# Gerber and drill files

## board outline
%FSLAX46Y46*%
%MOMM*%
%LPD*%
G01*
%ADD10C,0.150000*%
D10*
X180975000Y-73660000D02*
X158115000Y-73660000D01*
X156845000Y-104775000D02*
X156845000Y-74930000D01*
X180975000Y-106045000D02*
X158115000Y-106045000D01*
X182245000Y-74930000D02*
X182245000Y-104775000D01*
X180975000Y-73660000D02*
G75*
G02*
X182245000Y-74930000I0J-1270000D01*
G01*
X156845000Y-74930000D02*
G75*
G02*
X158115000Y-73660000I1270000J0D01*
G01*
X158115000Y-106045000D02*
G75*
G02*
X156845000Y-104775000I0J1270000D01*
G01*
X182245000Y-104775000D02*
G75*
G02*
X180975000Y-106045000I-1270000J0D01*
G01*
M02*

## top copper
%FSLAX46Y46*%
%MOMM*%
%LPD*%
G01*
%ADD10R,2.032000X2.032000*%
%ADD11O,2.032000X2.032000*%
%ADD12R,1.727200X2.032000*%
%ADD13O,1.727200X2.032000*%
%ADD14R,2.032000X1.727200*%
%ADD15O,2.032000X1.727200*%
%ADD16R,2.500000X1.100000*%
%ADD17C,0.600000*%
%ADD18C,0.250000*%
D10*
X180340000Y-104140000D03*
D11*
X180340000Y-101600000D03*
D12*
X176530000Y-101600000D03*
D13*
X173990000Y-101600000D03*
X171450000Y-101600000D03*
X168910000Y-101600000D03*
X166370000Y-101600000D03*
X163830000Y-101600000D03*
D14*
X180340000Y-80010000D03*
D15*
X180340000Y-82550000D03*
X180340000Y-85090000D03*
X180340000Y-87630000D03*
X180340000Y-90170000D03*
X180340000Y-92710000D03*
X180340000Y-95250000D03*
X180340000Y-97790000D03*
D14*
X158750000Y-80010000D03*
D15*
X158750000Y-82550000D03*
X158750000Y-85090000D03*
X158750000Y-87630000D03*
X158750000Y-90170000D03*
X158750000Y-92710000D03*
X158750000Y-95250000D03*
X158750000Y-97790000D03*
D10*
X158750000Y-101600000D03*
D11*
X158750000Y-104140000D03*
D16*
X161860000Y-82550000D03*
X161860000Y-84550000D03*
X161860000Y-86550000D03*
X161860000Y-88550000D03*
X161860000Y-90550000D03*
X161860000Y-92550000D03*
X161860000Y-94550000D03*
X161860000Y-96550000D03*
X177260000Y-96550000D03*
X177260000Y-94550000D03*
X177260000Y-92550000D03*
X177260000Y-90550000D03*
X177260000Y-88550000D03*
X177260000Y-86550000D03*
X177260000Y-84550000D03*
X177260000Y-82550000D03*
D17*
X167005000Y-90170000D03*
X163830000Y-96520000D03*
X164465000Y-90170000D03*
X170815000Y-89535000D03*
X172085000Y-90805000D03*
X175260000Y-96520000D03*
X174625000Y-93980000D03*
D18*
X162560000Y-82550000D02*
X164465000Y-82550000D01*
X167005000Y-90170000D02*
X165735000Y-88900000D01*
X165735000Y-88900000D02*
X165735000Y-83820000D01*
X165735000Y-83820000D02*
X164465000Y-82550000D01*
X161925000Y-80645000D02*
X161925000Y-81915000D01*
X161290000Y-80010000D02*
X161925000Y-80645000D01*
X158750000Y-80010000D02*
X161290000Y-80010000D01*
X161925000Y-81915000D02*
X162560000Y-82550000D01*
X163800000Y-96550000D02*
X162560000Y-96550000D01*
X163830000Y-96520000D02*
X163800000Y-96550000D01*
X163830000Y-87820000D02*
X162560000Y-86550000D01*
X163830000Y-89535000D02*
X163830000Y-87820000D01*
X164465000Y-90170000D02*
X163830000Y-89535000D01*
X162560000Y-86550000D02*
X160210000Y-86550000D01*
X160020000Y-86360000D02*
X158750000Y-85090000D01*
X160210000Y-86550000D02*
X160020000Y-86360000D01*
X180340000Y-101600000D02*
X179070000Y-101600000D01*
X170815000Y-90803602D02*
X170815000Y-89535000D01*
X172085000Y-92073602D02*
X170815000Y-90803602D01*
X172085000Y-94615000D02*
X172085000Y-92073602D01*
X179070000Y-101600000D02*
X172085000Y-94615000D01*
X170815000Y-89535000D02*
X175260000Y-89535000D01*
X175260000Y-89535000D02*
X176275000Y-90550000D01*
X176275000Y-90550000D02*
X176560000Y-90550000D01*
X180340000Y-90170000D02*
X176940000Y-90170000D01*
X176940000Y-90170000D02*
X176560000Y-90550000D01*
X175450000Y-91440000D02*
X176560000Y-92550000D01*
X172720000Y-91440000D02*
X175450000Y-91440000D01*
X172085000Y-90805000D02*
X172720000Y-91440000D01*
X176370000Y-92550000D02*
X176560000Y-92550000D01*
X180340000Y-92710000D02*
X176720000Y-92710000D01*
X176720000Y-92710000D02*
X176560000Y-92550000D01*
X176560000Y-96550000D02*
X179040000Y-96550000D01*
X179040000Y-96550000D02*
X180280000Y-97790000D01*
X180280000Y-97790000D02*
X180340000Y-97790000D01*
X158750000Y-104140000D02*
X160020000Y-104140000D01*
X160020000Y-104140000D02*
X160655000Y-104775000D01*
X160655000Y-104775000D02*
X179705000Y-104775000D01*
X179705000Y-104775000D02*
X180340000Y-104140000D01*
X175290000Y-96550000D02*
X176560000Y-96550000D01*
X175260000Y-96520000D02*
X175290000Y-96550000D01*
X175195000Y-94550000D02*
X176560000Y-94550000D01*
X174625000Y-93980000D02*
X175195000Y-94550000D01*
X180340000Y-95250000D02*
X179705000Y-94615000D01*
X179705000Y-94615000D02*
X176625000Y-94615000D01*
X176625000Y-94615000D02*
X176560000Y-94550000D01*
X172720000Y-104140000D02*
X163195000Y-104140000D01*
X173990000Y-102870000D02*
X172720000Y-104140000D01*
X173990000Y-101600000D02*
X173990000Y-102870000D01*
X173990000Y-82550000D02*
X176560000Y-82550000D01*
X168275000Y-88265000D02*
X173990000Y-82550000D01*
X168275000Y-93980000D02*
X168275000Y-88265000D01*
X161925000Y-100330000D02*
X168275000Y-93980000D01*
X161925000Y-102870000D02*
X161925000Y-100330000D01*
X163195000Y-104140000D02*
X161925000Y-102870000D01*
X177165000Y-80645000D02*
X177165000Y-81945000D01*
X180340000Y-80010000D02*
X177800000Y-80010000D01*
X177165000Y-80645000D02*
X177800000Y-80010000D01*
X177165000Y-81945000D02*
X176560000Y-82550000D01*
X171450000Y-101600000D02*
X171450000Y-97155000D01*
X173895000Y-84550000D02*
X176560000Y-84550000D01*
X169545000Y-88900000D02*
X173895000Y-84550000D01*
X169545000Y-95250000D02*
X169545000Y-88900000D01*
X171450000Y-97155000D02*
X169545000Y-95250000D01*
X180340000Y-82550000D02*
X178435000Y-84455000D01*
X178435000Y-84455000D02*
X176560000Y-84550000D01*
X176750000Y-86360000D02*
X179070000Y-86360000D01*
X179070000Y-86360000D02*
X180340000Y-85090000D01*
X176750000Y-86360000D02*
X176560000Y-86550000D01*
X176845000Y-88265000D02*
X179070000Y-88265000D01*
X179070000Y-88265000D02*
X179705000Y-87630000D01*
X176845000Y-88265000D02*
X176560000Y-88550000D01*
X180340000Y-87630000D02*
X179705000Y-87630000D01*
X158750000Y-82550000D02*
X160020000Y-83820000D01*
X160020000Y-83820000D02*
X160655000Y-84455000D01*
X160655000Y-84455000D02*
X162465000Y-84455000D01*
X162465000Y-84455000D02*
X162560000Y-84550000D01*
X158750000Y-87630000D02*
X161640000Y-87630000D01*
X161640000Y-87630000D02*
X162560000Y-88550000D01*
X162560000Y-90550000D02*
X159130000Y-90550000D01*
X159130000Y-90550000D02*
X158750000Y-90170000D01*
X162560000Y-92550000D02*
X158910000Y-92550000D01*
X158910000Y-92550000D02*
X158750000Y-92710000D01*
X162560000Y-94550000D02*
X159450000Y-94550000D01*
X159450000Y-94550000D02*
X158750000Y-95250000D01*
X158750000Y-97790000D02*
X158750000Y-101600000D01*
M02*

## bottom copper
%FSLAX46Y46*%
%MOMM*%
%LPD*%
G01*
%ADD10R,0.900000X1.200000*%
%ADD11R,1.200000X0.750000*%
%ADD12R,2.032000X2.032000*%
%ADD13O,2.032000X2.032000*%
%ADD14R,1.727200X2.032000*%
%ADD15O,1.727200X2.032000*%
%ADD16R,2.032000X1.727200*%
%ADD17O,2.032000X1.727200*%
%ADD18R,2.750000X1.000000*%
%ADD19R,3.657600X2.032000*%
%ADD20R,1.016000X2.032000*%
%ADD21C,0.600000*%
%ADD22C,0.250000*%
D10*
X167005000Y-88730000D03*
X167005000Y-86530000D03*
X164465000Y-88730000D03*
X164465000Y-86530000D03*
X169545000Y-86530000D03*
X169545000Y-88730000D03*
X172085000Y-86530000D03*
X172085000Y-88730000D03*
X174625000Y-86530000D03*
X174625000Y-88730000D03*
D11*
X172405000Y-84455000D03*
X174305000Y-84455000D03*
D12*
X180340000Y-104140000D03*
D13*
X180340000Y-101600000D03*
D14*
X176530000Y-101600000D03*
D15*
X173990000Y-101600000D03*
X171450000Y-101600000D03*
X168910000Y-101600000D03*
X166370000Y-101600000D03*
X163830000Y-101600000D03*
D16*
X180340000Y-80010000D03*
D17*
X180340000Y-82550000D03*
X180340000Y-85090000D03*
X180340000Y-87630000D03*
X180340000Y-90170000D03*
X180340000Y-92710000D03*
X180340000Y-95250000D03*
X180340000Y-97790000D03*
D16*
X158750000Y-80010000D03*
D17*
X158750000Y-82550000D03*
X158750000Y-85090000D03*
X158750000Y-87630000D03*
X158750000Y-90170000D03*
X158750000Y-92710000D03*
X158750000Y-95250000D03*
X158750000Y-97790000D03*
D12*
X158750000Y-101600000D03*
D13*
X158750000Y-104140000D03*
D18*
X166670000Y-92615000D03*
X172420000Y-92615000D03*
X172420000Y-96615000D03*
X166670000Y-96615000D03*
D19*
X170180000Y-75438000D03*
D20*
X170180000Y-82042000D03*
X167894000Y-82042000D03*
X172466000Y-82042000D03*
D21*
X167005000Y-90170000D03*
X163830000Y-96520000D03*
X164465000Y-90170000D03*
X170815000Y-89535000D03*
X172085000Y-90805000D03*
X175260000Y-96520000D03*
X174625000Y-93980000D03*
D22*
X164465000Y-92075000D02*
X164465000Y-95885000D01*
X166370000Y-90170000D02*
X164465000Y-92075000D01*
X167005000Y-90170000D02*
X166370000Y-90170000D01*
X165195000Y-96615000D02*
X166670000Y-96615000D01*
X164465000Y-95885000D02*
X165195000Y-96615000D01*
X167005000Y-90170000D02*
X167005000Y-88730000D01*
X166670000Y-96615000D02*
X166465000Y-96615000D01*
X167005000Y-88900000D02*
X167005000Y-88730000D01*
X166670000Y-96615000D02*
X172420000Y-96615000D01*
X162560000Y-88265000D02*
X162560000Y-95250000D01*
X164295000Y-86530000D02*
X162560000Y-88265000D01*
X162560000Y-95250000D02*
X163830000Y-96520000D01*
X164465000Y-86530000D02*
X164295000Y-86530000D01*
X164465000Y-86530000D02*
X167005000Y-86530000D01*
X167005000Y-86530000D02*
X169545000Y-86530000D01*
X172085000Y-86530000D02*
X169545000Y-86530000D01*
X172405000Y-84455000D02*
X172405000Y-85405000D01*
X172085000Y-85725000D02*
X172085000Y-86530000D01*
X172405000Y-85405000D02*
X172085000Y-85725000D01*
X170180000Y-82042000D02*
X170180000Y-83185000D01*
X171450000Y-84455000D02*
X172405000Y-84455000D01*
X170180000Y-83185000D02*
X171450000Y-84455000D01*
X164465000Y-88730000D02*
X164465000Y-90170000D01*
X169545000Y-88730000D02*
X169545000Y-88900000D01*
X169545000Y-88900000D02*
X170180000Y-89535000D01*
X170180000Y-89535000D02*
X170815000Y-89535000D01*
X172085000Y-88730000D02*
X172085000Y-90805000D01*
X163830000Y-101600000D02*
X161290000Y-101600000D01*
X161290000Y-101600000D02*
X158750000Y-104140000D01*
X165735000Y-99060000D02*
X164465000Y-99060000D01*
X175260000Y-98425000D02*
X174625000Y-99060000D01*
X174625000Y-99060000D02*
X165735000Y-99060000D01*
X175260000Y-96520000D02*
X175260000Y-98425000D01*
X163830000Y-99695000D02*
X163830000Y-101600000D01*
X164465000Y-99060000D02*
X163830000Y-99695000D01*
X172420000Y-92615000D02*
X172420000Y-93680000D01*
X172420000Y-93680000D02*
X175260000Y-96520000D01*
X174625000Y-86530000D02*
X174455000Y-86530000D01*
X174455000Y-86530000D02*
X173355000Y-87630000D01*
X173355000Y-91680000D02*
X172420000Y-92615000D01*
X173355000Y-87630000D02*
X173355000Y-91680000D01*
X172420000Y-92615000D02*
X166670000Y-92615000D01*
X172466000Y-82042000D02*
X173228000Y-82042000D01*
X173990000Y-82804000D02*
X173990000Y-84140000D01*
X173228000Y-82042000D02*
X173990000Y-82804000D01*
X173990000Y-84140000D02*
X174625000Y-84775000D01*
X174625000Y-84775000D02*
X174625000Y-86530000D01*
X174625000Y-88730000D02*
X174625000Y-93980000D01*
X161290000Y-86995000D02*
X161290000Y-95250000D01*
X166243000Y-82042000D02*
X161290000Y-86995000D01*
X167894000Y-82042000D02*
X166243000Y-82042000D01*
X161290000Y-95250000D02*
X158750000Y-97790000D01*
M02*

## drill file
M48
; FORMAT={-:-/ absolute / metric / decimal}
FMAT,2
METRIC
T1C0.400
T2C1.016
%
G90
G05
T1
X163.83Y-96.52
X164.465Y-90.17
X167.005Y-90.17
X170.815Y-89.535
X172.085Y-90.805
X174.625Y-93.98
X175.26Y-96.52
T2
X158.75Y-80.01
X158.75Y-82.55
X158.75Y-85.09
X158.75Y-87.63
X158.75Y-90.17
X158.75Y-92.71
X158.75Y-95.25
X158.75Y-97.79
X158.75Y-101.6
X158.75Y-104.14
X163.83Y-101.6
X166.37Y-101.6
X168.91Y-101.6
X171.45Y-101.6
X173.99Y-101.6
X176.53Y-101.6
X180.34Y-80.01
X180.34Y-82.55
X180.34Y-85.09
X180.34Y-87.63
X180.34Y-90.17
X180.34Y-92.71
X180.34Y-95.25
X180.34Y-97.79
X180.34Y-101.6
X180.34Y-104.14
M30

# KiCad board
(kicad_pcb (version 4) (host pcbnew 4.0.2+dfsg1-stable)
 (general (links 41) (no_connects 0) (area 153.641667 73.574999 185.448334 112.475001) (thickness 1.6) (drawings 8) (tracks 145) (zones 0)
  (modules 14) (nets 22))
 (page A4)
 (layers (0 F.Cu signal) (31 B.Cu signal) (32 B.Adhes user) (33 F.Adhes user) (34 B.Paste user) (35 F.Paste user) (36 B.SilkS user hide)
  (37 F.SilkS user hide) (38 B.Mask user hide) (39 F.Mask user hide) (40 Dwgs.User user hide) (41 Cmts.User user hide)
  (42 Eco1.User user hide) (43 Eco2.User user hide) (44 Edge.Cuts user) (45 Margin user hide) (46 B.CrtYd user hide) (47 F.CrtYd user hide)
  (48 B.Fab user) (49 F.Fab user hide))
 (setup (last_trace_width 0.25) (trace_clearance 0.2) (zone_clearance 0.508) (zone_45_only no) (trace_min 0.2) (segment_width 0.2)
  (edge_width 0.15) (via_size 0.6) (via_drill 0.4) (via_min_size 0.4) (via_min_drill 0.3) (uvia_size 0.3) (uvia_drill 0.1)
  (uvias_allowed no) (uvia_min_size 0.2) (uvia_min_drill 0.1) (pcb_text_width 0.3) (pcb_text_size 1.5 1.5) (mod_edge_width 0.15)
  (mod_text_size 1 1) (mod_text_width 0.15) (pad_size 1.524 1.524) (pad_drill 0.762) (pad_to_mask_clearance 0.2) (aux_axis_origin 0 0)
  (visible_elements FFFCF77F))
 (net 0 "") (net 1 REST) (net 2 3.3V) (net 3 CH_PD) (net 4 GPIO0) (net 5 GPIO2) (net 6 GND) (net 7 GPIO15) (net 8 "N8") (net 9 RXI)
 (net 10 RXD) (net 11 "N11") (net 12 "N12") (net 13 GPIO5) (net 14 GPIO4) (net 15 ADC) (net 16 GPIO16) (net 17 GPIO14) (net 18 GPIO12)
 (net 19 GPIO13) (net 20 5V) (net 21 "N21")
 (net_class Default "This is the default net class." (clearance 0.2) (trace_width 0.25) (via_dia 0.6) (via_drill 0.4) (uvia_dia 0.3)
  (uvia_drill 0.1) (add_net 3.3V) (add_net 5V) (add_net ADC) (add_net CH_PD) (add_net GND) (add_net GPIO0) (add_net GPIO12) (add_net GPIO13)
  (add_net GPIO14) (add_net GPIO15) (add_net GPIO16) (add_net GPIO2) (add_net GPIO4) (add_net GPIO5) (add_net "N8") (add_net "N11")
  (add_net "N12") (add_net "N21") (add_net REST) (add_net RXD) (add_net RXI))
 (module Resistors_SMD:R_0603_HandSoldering (layer B.Cu) (at 167.005 87.63 90)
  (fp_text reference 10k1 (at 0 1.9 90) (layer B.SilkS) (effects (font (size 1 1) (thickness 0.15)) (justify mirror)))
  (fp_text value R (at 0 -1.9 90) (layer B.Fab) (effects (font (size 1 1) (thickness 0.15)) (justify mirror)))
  (pad 1 smd rect (at -1.1 0 90) (size 1.2 0.9) (layers B.Cu B.Paste B.Mask) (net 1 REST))
  (pad 2 smd rect (at 1.1 0 90) (size 1.2 0.9) (layers B.Cu B.Paste B.Mask) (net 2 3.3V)))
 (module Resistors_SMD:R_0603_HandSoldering (layer B.Cu) (at 164.465 87.63 90)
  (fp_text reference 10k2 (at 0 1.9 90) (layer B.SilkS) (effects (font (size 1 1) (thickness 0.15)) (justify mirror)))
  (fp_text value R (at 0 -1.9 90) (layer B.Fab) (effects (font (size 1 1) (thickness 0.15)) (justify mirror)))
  (pad 1 smd rect (at -1.1 0 90) (size 1.2 0.9) (layers B.Cu B.Paste B.Mask) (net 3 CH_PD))
  (pad 2 smd rect (at 1.1 0 90) (size 1.2 0.9) (layers B.Cu B.Paste B.Mask) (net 2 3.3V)))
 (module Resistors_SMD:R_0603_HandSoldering (layer B.Cu) (at 169.545 87.63 270)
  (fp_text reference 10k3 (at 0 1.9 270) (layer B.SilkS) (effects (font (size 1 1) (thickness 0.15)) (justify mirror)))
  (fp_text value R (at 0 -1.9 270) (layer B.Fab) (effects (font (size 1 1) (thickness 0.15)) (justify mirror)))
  (pad 1 smd rect (at -1.1 0 270) (size 1.2 0.9) (layers B.Cu B.Paste B.Mask) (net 2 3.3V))
  (pad 2 smd rect (at 1.1 0 270) (size 1.2 0.9) (layers B.Cu B.Paste B.Mask) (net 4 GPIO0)))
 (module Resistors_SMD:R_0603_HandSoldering (layer B.Cu) (at 172.085 87.63 270)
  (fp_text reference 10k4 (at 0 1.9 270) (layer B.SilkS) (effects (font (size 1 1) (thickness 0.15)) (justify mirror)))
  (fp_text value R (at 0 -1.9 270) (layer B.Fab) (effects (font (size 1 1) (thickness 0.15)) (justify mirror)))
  (pad 1 smd rect (at -1.1 0 270) (size 1.2 0.9) (layers B.Cu B.Paste B.Mask) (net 2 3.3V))
  (pad 2 smd rect (at 1.1 0 270) (size 1.2 0.9) (layers B.Cu B.Paste B.Mask) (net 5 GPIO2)))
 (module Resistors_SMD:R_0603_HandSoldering (layer B.Cu) (at 174.625 87.63 270)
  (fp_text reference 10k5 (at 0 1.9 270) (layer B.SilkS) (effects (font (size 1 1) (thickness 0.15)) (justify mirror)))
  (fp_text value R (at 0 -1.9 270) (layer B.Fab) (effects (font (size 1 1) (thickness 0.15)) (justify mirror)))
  (pad 1 smd rect (at -1.1 0 270) (size 1.2 0.9) (layers B.Cu B.Paste B.Mask) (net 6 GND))
  (pad 2 smd rect (at 1.1 0 270) (size 1.2 0.9) (layers B.Cu B.Paste B.Mask) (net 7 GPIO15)))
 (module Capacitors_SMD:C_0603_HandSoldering (layer B.Cu) (at 173.355 84.455)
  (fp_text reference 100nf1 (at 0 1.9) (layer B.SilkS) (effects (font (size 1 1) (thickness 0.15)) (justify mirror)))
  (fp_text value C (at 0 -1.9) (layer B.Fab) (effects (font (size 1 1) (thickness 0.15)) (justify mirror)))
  (pad 1 smd rect (at -0.95 0) (size 1.2 0.75) (layers B.Cu B.Paste B.Mask) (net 2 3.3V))
  (pad 2 smd rect (at 0.95 0) (size 1.2 0.75) (layers B.Cu B.Paste B.Mask) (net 6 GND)))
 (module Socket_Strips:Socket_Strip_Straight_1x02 (layer F.Cu) (at 180.34 104.14 90)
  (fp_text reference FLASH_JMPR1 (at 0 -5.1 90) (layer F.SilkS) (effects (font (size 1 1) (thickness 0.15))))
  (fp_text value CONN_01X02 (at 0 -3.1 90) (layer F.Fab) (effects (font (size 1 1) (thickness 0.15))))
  (pad 1 thru_hole rect (at 0 0 90) (size 2.032 2.032) (drill 1.016) (layers *.Cu *.Mask F.SilkS) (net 6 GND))
  (pad 2 thru_hole oval (at 2.54 0 90) (size 2.032 2.032) (drill 1.016) (layers *.Cu *.Mask F.SilkS) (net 4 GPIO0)))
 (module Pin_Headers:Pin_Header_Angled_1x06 (layer F.Cu) (at 176.53 101.6 270)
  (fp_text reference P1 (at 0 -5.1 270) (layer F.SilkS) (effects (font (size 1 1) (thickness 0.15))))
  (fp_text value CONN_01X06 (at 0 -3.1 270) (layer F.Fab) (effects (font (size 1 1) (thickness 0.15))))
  (pad 1 thru_hole rect (at 0 0 270) (size 2.032 1.7272) (drill 1.016) (layers *.Cu *.Mask F.SilkS) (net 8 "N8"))
  (pad 2 thru_hole oval (at 0 2.54 270) (size 2.032 1.7272) (drill 1.016) (layers *.Cu *.Mask F.SilkS) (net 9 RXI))
  (pad 3 thru_hole oval (at 0 5.08 270) (size 2.032 1.7272) (drill 1.016) (layers *.Cu *.Mask F.SilkS) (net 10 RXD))
  (pad 4 thru_hole oval (at 0 7.62 270) (size 2.032 1.7272) (drill 1.016) (layers *.Cu *.Mask F.SilkS) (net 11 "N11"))
  (pad 5 thru_hole oval (at 0 10.16 270) (size 2.032 1.7272) (drill 1.016) (layers *.Cu *.Mask F.SilkS) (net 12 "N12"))
  (pad 6 thru_hole oval (at 0 12.7 270) (size 2.032 1.7272) (drill 1.016) (layers *.Cu *.Mask F.SilkS) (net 6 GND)))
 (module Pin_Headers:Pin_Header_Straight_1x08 (layer F.Cu) (at 180.34 80.01)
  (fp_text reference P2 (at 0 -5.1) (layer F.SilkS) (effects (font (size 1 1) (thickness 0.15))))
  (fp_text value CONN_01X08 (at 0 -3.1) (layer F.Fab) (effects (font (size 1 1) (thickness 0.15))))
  (pad 1 thru_hole rect (at 0 0) (size 2.032 1.7272) (drill 1.016) (layers *.Cu *.Mask F.SilkS) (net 9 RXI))
  (pad 2 thru_hole oval (at 0 2.54) (size 2.032 1.7272) (drill 1.016) (layers *.Cu *.Mask F.SilkS) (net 10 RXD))
  (pad 3 thru_hole oval (at 0 5.08) (size 2.032 1.7272) (drill 1.016) (layers *.Cu *.Mask F.SilkS) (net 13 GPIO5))
  (pad 4 thru_hole oval (at 0 7.62) (size 2.032 1.7272) (drill 1.016) (layers *.Cu *.Mask F.SilkS) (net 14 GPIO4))
  (pad 5 thru_hole oval (at 0 10.16) (size 2.032 1.7272) (drill 1.016) (layers *.Cu *.Mask F.SilkS) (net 4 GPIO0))
  (pad 6 thru_hole oval (at 0 12.7) (size 2.032 1.7272) (drill 1.016) (layers *.Cu *.Mask F.SilkS) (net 5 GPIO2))
  (pad 7 thru_hole oval (at 0 15.24) (size 2.032 1.7272) (drill 1.016) (layers *.Cu *.Mask F.SilkS) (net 7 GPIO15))
  (pad 8 thru_hole oval (at 0 17.78) (size 2.032 1.7272) (drill 1.016) (layers *.Cu *.Mask F.SilkS) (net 6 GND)))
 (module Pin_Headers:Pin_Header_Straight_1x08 (layer F.Cu) (at 158.75 80.01)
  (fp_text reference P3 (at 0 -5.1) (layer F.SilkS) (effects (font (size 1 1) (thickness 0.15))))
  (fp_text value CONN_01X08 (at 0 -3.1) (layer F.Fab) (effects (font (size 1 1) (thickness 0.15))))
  (pad 1 thru_hole rect (at 0 0) (size 2.032 1.7272) (drill 1.016) (layers *.Cu *.Mask F.SilkS) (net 1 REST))
  (pad 2 thru_hole oval (at 0 2.54) (size 2.032 1.7272) (drill 1.016) (layers *.Cu *.Mask F.SilkS) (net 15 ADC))
  (pad 3 thru_hole oval (at 0 5.08) (size 2.032 1.7272) (drill 1.016) (layers *.Cu *.Mask F.SilkS) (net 3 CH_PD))
  (pad 4 thru_hole oval (at 0 7.62) (size 2.032 1.7272) (drill 1.016) (layers *.Cu *.Mask F.SilkS) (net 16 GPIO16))
  (pad 5 thru_hole oval (at 0 10.16) (size 2.032 1.7272) (drill 1.016) (layers *.Cu *.Mask F.SilkS) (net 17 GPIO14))
  (pad 6 thru_hole oval (at 0 12.7) (size 2.032 1.7272) (drill 1.016) (layers *.Cu *.Mask F.SilkS) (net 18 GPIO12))
  (pad 7 thru_hole oval (at 0 15.24) (size 2.032 1.7272) (drill 1.016) (layers *.Cu *.Mask F.SilkS) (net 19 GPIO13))
  (pad 8 thru_hole oval (at 0 17.78) (size 2.032 1.7272) (drill 1.016) (layers *.Cu *.Mask F.SilkS) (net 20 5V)))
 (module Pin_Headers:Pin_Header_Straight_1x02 (layer F.Cu) (at 158.75 101.6)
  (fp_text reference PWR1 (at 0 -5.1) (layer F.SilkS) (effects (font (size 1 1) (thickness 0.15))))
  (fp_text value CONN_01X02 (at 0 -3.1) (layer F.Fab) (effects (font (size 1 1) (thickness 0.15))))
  (pad 1 thru_hole rect (at 0 0) (size 2.032 2.032) (drill 1.016) (layers *.Cu *.Mask F.SilkS) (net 20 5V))
  (pad 2 thru_hole oval (at 0 2.54) (size 2.032 2.032) (drill 1.016) (layers *.Cu *.Mask F.SilkS) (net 6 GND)))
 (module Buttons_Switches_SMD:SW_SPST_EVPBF (layer B.Cu) (at 169.545 94.615 180)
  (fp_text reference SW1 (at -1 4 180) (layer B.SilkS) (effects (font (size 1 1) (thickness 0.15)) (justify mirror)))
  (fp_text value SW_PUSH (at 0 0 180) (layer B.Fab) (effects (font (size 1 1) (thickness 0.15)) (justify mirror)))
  (pad 1 smd rect (at 2.875 2 180) (size 2.75 1) (layers B.Cu B.Paste B.Mask) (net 6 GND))
  (pad 1 smd rect (at -2.875 2 180) (size 2.75 1) (layers B.Cu B.Paste B.Mask) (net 6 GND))
  (pad 2 smd rect (at -2.875 -2 180) (size 2.75 1) (layers B.Cu B.Paste B.Mask) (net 1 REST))
  (pad 2 smd rect (at 2.875 -2 180) (size 2.75 1) (layers B.Cu B.Paste B.Mask) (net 1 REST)))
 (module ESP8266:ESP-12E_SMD (layer F.Cu) (at 162.56 82.55)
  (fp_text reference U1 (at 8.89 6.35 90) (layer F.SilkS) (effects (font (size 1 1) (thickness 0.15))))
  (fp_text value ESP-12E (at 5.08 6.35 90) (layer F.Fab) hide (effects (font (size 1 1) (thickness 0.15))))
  (pad 1 smd rect (at 0 0) (size 2.5 1.1) (drill (offset -0.7 0)) (layers F.Cu F.Paste F.Mask) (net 1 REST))
  (pad 2 smd rect (at 0 2) (size 2.5 1.1) (drill (offset -0.7 0)) (layers F.Cu F.Paste F.Mask) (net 15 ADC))
  (pad 3 smd rect (at 0 4) (size 2.5 1.1) (drill (offset -0.7 0)) (layers F.Cu F.Paste F.Mask) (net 3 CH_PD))
  (pad 4 smd rect (at 0 6) (size 2.5 1.1) (drill (offset -0.7 0)) (layers F.Cu F.Paste F.Mask) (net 16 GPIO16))
  (pad 5 smd rect (at 0 8) (size 2.5 1.1) (drill (offset -0.7 0)) (layers F.Cu F.Paste F.Mask) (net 17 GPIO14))
  (pad 6 smd rect (at 0 10) (size 2.5 1.1) (drill (offset -0.7 0)) (layers F.Cu F.Paste F.Mask) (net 18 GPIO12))
  (pad 7 smd rect (at 0 12) (size 2.5 1.1) (drill (offset -0.7 0)) (layers F.Cu F.Paste F.Mask) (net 19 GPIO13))
  (pad 8 smd rect (at 0 14) (size 2.5 1.1) (drill (offset -0.7 0)) (layers F.Cu F.Paste F.Mask) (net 2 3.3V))
  (pad 9 smd rect (at 14 14) (size 2.5 1.1) (drill (offset 0.7 0)) (layers F.Cu F.Paste F.Mask) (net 6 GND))
  (pad 10 smd rect (at 14 12) (size 2.5 1.1) (drill (offset 0.7 0)) (layers F.Cu F.Paste F.Mask) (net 7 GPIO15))
  (pad 11 smd rect (at 14 10) (size 2.5 1.1) (drill (offset 0.7 0)) (layers F.Cu F.Paste F.Mask) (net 5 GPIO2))
  (pad 12 smd rect (at 14 8) (size 2.5 1.1) (drill (offset 0.7 0)) (layers F.Cu F.Paste F.Mask) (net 4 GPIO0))
  (pad 13 smd rect (at 14 6) (size 2.5 1.1) (drill (offset 0.7 0)) (layers F.Cu F.Paste F.Mask) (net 14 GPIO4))
  (pad 14 smd rect (at 14 4) (size 2.5 1.1) (drill (offset 0.7 0)) (layers F.Cu F.Paste F.Mask) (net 13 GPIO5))
  (pad 15 smd rect (at 14 2) (size 2.5 1.1) (drill (offset 0.7 0)) (layers F.Cu F.Paste F.Mask) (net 10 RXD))
  (pad 16 smd rect (at 14 0) (size 2.5 1.1) (drill (offset 0.7 0)) (layers F.Cu F.Paste F.Mask) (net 9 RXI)))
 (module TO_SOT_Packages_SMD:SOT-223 (layer B.Cu) (at 170.18 78.74 180)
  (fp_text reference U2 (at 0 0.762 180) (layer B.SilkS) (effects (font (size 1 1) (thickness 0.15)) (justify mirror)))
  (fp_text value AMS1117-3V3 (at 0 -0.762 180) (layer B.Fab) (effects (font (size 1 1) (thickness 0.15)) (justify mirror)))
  (pad 4 smd rect (at 0 3.302 180) (size 3.6576 2.032) (layers B.Cu B.Paste B.Mask) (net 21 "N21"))
  (pad 2 smd rect (at 0 -3.302 180) (size 1.016 2.032) (layers B.Cu B.Paste B.Mask) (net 2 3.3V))
  (pad 3 smd rect (at 2.286 -3.302 180) (size 1.016 2.032) (layers B.Cu B.Paste B.Mask) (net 20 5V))
  (pad 1 smd rect (at -2.286 -3.302 180) (size 1.016 2.032) (layers B.Cu B.Paste B.Mask) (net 6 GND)))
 (gr_line (start 180.975 73.66) (end 158.115 73.66) (angle 90) (layer Edge.Cuts) (width 0.15))
 (gr_line (start 156.845 104.775) (end 156.845 74.93) (angle 90) (layer Edge.Cuts) (width 0.15))
 (gr_line (start 180.975 106.045) (end 158.115 106.045) (angle 90) (layer Edge.Cuts) (width 0.15))
 (gr_line (start 182.245 74.93) (end 182.245 104.775) (angle 90) (layer Edge.Cuts) (width 0.15))
 (gr_arc (start 180.975 74.93) (end 180.975 73.66) (angle 90) (layer Edge.Cuts) (width 0.15))
 (gr_arc (start 158.115 74.93) (end 156.845 74.93) (angle 90) (layer Edge.Cuts) (width 0.15))
 (gr_arc (start 158.115 104.775) (end 158.115 106.045) (angle 90) (layer Edge.Cuts) (width 0.15))
 (gr_arc (start 180.975 104.775) (end 182.245 104.775) (angle 90) (layer Edge.Cuts) (width 0.15))
 (segment (start 164.465 92.075) (end 164.465 95.885) (width 0.25) (layer B.Cu) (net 1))
 (segment (start 166.37 90.17) (end 164.465 92.075) (width 0.25) (layer B.Cu) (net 1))
 (segment (start 167.005 90.17) (end 166.37 90.17) (width 0.25) (layer B.Cu) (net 1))
 (segment (start 165.195 96.615) (end 166.67 96.615) (width 0.25) (layer B.Cu) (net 1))
 (segment (start 164.465 95.885) (end 165.195 96.615) (width 0.25) (layer B.Cu) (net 1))
 (segment (start 162.56 82.55) (end 164.465 82.55) (width 0.25) (layer F.Cu) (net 1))
 (via (at 167.005 90.17) (size 0.6) (drill 0.4) (layers F.Cu B.Cu) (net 1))
 (segment (start 167.005 90.17) (end 165.735 88.9) (width 0.25) (layer F.Cu) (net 1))
 (segment (start 165.735 88.9) (end 165.735 83.82) (width 0.25) (layer F.Cu) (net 1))
 (segment (start 165.735 83.82) (end 164.465 82.55) (width 0.25) (layer F.Cu) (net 1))
 (segment (start 167.005 90.17) (end 167.005 88.73) (width 0.25) (layer B.Cu) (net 1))
 (segment (start 166.67 96.615) (end 166.465 96.615) (width 0.25) (layer B.Cu) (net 1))
 (segment (start 167.005 88.9) (end 167.005 88.73) (width 0.25) (layer B.Cu) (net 1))
 (segment (start 166.67 96.615) (end 172.42 96.615) (width 0.25) (layer B.Cu) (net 1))
 (segment (start 161.925 80.645) (end 161.925 81.915) (width 0.25) (layer F.Cu) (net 1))
 (segment (start 161.29 80.01) (end 161.925 80.645) (width 0.25) (layer F.Cu) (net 1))
 (segment (start 158.75 80.01) (end 161.29 80.01) (width 0.25) (layer F.Cu) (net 1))
 (segment (start 161.925 81.915) (end 162.56 82.55) (width 0.25) (layer F.Cu) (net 1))
 (segment (start 162.56 88.265) (end 162.56 95.25) (width 0.25) (layer B.Cu) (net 2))
 (segment (start 164.295 86.53) (end 162.56 88.265) (width 0.25) (layer B.Cu) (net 2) (status 400000))
 (segment (start 163.8 96.55) (end 162.56 96.55) (width 0.25) (layer F.Cu) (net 2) (status 800000))
 (segment (start 163.83 96.52) (end 163.8 96.55) (width 0.25) (layer F.Cu) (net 2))
 (via (at 163.83 96.52) (size 0.6) (drill 0.4) (layers F.Cu B.Cu) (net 2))
 (segment (start 162.56 95.25) (end 163.83 96.52) (width 0.25) (layer B.Cu) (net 2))
 (segment (start 164.465 86.53) (end 164.295 86.53) (width 0.25) (layer B.Cu) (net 2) (status C00000))
 (segment (start 164.465 86.53) (end 167.005 86.53) (width 0.25) (layer B.Cu) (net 2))
 (segment (start 167.005 86.53) (end 169.545 86.53) (width 0.25) (layer B.Cu) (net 2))
 (segment (start 172.085 86.53) (end 169.545 86.53) (width 0.25) (layer B.Cu) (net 2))
 (segment (start 172.405 84.455) (end 172.405 85.405) (width 0.25) (layer B.Cu) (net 2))
 (segment (start 172.085 85.725) (end 172.085 86.53) (width 0.25) (layer B.Cu) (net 2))
 (segment (start 172.405 85.405) (end 172.085 85.725) (width 0.25) (layer B.Cu) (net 2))
 (segment (start 170.18 82.042) (end 170.18 83.185) (width 0.25) (layer B.Cu) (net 2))
 (segment (start 171.45 84.455) (end 172.405 84.455) (width 0.25) (layer B.Cu) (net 2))
 (segment (start 170.18 83.185) (end 171.45 84.455) (width 0.25) (layer B.Cu) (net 2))
 (segment (start 164.465 88.73) (end 164.465 90.17) (width 0.25) (layer B.Cu) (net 3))
 (segment (start 163.83 87.82) (end 162.56 86.55) (width 0.25) (layer F.Cu) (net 3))
 (segment (start 163.83 89.535) (end 163.83 87.82) (width 0.25) (layer F.Cu) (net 3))
 (segment (start 164.465 90.17) (end 163.83 89.535) (width 0.25) (layer F.Cu) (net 3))
 (via (at 164.465 90.17) (size 0.6) (drill 0.4) (layers F.Cu B.Cu) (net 3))
 (segment (start 162.56 86.55) (end 160.21 86.55) (width 0.25) (layer F.Cu) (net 3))
 (segment (start 160.02 86.36) (end 158.75 85.09) (width 0.25) (layer F.Cu) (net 3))
 (segment (start 160.21 86.55) (end 160.02 86.36) (width 0.25) (layer F.Cu) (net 3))
 (segment (start 180.34 101.6) (end 179.07 101.6) (width 0.25) (layer F.Cu) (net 4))
 (segment (start 170.815 90.803602) (end 170.815 89.535) (width 0.25) (layer F.Cu) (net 4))
 (segment (start 172.085 92.073602) (end 170.815 90.803602) (width 0.25) (layer F.Cu) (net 4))
 (segment (start 172.085 94.615) (end 172.085 92.073602) (width 0.25) (layer F.Cu) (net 4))
 (segment (start 179.07 101.6) (end 172.085 94.615) (width 0.25) (layer F.Cu) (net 4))
 (segment (start 169.545 88.73) (end 169.545 88.9) (width 0.25) (layer B.Cu) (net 4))
 (segment (start 169.545 88.9) (end 170.18 89.535) (width 0.25) (layer B.Cu) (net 4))
 (segment (start 170.18 89.535) (end 170.815 89.535) (width 0.25) (layer B.Cu) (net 4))
 (via (at 170.815 89.535) (size 0.6) (drill 0.4) (layers F.Cu B.Cu) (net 4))
 (segment (start 170.815 89.535) (end 175.26 89.535) (width 0.25) (layer F.Cu) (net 4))
 (segment (start 175.26 89.535) (end 176.275 90.55) (width 0.25) (layer F.Cu) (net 4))
 (segment (start 176.275 90.55) (end 176.56 90.55) (width 0.25) (layer F.Cu) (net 4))
 (segment (start 180.34 90.17) (end 176.94 90.17) (width 0.25) (layer F.Cu) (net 4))
 (segment (start 176.94 90.17) (end 176.56 90.55) (width 0.25) (layer F.Cu) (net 4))
 (segment (start 172.085 88.73) (end 172.085 90.805) (width 0.25) (layer B.Cu) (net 5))
 (segment (start 175.45 91.44) (end 176.56 92.55) (width 0.25) (layer F.Cu) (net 5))
 (segment (start 172.72 91.44) (end 175.45 91.44) (width 0.25) (layer F.Cu) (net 5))
 (segment (start 172.085 90.805) (end 172.72 91.44) (width 0.25) (layer F.Cu) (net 5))
 (via (at 172.085 90.805) (size 0.6) (drill 0.4) (layers F.Cu B.Cu) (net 5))
 (segment (start 176.37 92.55) (end 176.56 92.55) (width 0.25) (layer F.Cu) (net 5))
 (segment (start 180.34 92.71) (end 176.72 92.71) (width 0.25) (layer F.Cu) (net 5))
 (segment (start 176.72 92.71) (end 176.56 92.55) (width 0.25) (layer F.Cu) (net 5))
 (segment (start 176.56 96.55) (end 179.04 96.55) (width 0.25) (layer F.Cu) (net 6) (status 400000))
 (segment (start 179.04 96.55) (end 180.28 97.79) (width 0.25) (layer F.Cu) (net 6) (status 800000))
 (segment (start 180.28 97.79) (end 180.34 97.79) (width 0.25) (layer F.Cu) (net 6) (status C00000))
 (segment (start 163.83 101.6) (end 161.29 101.6) (width 0.25) (layer B.Cu) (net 6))
 (segment (start 161.29 101.6) (end 158.75 104.14) (width 0.25) (layer B.Cu) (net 6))
 (segment (start 165.735 99.06) (end 164.465 99.06) (width 0.25) (layer B.Cu) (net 6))
 (segment (start 175.26 98.425) (end 174.625 99.06) (width 0.25) (layer B.Cu) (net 6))
 (segment (start 174.625 99.06) (end 165.735 99.06) (width 0.25) (layer B.Cu) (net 6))
 (segment (start 175.26 96.52) (end 175.26 98.425) (width 0.25) (layer B.Cu) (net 6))
 (segment (start 163.83 99.695) (end 163.83 101.6) (width 0.25) (layer B.Cu) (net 6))
 (segment (start 164.465 99.06) (end 163.83 99.695) (width 0.25) (layer B.Cu) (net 6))
 (segment (start 158.75 104.14) (end 160.02 104.14) (width 0.25) (layer F.Cu) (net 6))
 (segment (start 160.02 104.14) (end 160.655 104.775) (width 0.25) (layer F.Cu) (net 6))
 (segment (start 160.655 104.775) (end 179.705 104.775) (width 0.25) (layer F.Cu) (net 6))
 (segment (start 179.705 104.775) (end 180.34 104.14) (width 0.25) (layer F.Cu) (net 6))
 (segment (start 172.42 92.615) (end 172.42 93.68) (width 0.25) (layer B.Cu) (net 6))
 (segment (start 175.29 96.55) (end 176.56 96.55) (width 0.25) (layer F.Cu) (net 6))
 (segment (start 175.26 96.52) (end 175.29 96.55) (width 0.25) (layer F.Cu) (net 6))
 (via (at 175.26 96.52) (size 0.6) (drill 0.4) (layers F.Cu B.Cu) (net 6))
 (segment (start 172.42 93.68) (end 175.26 96.52) (width 0.25) (layer B.Cu) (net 6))
 (segment (start 174.625 86.53) (end 174.455 86.53) (width 0.25) (layer B.Cu) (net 6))
 (segment (start 174.455 86.53) (end 173.355 87.63) (width 0.25) (layer B.Cu) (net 6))
 (segment (start 173.355 91.68) (end 172.42 92.615) (width 0.25) (layer B.Cu) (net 6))
 (segment (start 173.355 87.63) (end 173.355 91.68) (width 0.25) (layer B.Cu) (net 6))
 (segment (start 172.42 92.615) (end 166.67 92.615) (width 0.25) (layer B.Cu) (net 6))
 (segment (start 172.466 82.042) (end 173.228 82.042) (width 0.25) (layer B.Cu) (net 6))
 (segment (start 173.99 82.804) (end 173.99 84.14) (width 0.25) (layer B.Cu) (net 6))
 (segment (start 173.228 82.042) (end 173.99 82.804) (width 0.25) (layer B.Cu) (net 6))
 (segment (start 173.99 84.14) (end 174.625 84.775) (width 0.25) (layer B.Cu) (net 6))
 (segment (start 174.625 84.775) (end 174.625 86.53) (width 0.25) (layer B.Cu) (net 6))
 (segment (start 174.625 88.73) (end 174.625 93.98) (width 0.25) (layer B.Cu) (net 7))
 (segment (start 175.195 94.55) (end 176.56 94.55) (width 0.25) (layer F.Cu) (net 7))
 (segment (start 174.625 93.98) (end 175.195 94.55) (width 0.25) (layer F.Cu) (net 7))
 (via (at 174.625 93.98) (size 0.6) (drill 0.4) (layers F.Cu B.Cu) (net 7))
 (segment (start 180.34 95.25) (end 179.705 94.615) (width 0.25) (layer F.Cu) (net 7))
 (segment (start 179.705 94.615) (end 176.625 94.615) (width 0.25) (layer F.Cu) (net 7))
 (segment (start 176.625 94.615) (end 176.56 94.55) (width 0.25) (layer F.Cu) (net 7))
 (segment (start 172.72 104.14) (end 163.195 104.14) (width 0.25) (layer F.Cu) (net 9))
 (segment (start 173.99 102.87) (end 172.72 104.14) (width 0.25) (layer F.Cu) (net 9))
 (segment (start 173.99 101.6) (end 173.99 102.87) (width 0.25) (layer F.Cu) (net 9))
 (segment (start 173.99 82.55) (end 176.56 82.55) (width 0.25) (layer F.Cu) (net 9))
 (segment (start 168.275 88.265) (end 173.99 82.55) (width 0.25) (layer F.Cu) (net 9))
 (segment (start 168.275 93.98) (end 168.275 88.265) (width 0.25) (layer F.Cu) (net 9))
 (segment (start 161.925 100.33) (end 168.275 93.98) (width 0.25) (layer F.Cu) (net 9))
 (segment (start 161.925 102.87) (end 161.925 100.33) (width 0.25) (layer F.Cu) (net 9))
 (segment (start 163.195 104.14) (end 161.925 102.87) (width 0.25) (layer F.Cu) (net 9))
 (segment (start 177.165 80.645) (end 177.165 81.945) (width 0.25) (layer F.Cu) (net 9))
 (segment (start 180.34 80.01) (end 177.8 80.01) (width 0.25) (layer F.Cu) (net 9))
 (segment (start 177.165 80.645) (end 177.8 80.01) (width 0.25) (layer F.Cu) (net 9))
 (segment (start 177.165 81.945) (end 176.56 82.55) (width 0.25) (layer F.Cu) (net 9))
 (segment (start 171.45 101.6) (end 171.45 97.155) (width 0.25) (layer F.Cu) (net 10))
 (segment (start 173.895 84.55) (end 176.56 84.55) (width 0.25) (layer F.Cu) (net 10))
 (segment (start 169.545 88.9) (end 173.895 84.55) (width 0.25) (layer F.Cu) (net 10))
 (segment (start 169.545 95.25) (end 169.545 88.9) (width 0.25) (layer F.Cu) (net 10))
 (segment (start 171.45 97.155) (end 169.545 95.25) (width 0.25) (layer F.Cu) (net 10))
 (segment (start 180.34 82.55) (end 178.435 84.455) (width 0.25) (layer F.Cu) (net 10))
 (segment (start 178.435 84.455) (end 176.56 84.55) (width 0.25) (layer F.Cu) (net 10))
 (segment (start 176.75 86.36) (end 179.07 86.36) (width 0.25) (layer F.Cu) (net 13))
 (segment (start 179.07 86.36) (end 180.34 85.09) (width 0.25) (layer F.Cu) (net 13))
 (segment (start 176.75 86.36) (end 176.56 86.55) (width 0.25) (layer F.Cu) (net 13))
 (segment (start 176.845 88.265) (end 179.07 88.265) (width 0.25) (layer F.Cu) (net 14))
 (segment (start 179.07 88.265) (end 179.705 87.63) (width 0.25) (layer F.Cu) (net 14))
 (segment (start 176.845 88.265) (end 176.56 88.55) (width 0.25) (layer F.Cu) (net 14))
 (segment (start 180.34 87.63) (end 179.705 87.63) (width 0.25) (layer F.Cu) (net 14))
 (segment (start 158.75 82.55) (end 160.02 83.82) (width 0.25) (layer F.Cu) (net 15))
 (segment (start 160.02 83.82) (end 160.655 84.455) (width 0.25) (layer F.Cu) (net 15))
 (segment (start 160.655 84.455) (end 162.465 84.455) (width 0.25) (layer F.Cu) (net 15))
 (segment (start 162.465 84.455) (end 162.56 84.55) (width 0.25) (layer F.Cu) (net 15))
 (segment (start 158.75 87.63) (end 161.64 87.63) (width 0.25) (layer F.Cu) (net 16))
 (segment (start 161.64 87.63) (end 162.56 88.55) (width 0.25) (layer F.Cu) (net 16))
 (segment (start 162.56 90.55) (end 159.13 90.55) (width 0.25) (layer F.Cu) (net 17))
 (segment (start 159.13 90.55) (end 158.75 90.17) (width 0.25) (layer F.Cu) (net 17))
 (segment (start 162.56 92.55) (end 158.91 92.55) (width 0.25) (layer F.Cu) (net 18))
 (segment (start 158.91 92.55) (end 158.75 92.71) (width 0.25) (layer F.Cu) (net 18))
 (segment (start 162.56 94.55) (end 159.45 94.55) (width 0.25) (layer F.Cu) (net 19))
 (segment (start 159.45 94.55) (end 158.75 95.25) (width 0.25) (layer F.Cu) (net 19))
 (segment (start 161.29 86.995) (end 161.29 95.25) (width 0.25) (layer B.Cu) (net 20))
 (segment (start 166.243 82.042) (end 161.29 86.995) (width 0.25) (layer B.Cu) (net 20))
 (segment (start 167.894 82.042) (end 166.243 82.042) (width 0.25) (layer B.Cu) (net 20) (status 400000))
 (segment (start 161.29 95.25) (end 158.75 97.79) (width 0.25) (layer B.Cu) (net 20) (status 800000))
 (segment (start 158.75 97.79) (end 158.75 101.6) (width 0.25) (layer F.Cu) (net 20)))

